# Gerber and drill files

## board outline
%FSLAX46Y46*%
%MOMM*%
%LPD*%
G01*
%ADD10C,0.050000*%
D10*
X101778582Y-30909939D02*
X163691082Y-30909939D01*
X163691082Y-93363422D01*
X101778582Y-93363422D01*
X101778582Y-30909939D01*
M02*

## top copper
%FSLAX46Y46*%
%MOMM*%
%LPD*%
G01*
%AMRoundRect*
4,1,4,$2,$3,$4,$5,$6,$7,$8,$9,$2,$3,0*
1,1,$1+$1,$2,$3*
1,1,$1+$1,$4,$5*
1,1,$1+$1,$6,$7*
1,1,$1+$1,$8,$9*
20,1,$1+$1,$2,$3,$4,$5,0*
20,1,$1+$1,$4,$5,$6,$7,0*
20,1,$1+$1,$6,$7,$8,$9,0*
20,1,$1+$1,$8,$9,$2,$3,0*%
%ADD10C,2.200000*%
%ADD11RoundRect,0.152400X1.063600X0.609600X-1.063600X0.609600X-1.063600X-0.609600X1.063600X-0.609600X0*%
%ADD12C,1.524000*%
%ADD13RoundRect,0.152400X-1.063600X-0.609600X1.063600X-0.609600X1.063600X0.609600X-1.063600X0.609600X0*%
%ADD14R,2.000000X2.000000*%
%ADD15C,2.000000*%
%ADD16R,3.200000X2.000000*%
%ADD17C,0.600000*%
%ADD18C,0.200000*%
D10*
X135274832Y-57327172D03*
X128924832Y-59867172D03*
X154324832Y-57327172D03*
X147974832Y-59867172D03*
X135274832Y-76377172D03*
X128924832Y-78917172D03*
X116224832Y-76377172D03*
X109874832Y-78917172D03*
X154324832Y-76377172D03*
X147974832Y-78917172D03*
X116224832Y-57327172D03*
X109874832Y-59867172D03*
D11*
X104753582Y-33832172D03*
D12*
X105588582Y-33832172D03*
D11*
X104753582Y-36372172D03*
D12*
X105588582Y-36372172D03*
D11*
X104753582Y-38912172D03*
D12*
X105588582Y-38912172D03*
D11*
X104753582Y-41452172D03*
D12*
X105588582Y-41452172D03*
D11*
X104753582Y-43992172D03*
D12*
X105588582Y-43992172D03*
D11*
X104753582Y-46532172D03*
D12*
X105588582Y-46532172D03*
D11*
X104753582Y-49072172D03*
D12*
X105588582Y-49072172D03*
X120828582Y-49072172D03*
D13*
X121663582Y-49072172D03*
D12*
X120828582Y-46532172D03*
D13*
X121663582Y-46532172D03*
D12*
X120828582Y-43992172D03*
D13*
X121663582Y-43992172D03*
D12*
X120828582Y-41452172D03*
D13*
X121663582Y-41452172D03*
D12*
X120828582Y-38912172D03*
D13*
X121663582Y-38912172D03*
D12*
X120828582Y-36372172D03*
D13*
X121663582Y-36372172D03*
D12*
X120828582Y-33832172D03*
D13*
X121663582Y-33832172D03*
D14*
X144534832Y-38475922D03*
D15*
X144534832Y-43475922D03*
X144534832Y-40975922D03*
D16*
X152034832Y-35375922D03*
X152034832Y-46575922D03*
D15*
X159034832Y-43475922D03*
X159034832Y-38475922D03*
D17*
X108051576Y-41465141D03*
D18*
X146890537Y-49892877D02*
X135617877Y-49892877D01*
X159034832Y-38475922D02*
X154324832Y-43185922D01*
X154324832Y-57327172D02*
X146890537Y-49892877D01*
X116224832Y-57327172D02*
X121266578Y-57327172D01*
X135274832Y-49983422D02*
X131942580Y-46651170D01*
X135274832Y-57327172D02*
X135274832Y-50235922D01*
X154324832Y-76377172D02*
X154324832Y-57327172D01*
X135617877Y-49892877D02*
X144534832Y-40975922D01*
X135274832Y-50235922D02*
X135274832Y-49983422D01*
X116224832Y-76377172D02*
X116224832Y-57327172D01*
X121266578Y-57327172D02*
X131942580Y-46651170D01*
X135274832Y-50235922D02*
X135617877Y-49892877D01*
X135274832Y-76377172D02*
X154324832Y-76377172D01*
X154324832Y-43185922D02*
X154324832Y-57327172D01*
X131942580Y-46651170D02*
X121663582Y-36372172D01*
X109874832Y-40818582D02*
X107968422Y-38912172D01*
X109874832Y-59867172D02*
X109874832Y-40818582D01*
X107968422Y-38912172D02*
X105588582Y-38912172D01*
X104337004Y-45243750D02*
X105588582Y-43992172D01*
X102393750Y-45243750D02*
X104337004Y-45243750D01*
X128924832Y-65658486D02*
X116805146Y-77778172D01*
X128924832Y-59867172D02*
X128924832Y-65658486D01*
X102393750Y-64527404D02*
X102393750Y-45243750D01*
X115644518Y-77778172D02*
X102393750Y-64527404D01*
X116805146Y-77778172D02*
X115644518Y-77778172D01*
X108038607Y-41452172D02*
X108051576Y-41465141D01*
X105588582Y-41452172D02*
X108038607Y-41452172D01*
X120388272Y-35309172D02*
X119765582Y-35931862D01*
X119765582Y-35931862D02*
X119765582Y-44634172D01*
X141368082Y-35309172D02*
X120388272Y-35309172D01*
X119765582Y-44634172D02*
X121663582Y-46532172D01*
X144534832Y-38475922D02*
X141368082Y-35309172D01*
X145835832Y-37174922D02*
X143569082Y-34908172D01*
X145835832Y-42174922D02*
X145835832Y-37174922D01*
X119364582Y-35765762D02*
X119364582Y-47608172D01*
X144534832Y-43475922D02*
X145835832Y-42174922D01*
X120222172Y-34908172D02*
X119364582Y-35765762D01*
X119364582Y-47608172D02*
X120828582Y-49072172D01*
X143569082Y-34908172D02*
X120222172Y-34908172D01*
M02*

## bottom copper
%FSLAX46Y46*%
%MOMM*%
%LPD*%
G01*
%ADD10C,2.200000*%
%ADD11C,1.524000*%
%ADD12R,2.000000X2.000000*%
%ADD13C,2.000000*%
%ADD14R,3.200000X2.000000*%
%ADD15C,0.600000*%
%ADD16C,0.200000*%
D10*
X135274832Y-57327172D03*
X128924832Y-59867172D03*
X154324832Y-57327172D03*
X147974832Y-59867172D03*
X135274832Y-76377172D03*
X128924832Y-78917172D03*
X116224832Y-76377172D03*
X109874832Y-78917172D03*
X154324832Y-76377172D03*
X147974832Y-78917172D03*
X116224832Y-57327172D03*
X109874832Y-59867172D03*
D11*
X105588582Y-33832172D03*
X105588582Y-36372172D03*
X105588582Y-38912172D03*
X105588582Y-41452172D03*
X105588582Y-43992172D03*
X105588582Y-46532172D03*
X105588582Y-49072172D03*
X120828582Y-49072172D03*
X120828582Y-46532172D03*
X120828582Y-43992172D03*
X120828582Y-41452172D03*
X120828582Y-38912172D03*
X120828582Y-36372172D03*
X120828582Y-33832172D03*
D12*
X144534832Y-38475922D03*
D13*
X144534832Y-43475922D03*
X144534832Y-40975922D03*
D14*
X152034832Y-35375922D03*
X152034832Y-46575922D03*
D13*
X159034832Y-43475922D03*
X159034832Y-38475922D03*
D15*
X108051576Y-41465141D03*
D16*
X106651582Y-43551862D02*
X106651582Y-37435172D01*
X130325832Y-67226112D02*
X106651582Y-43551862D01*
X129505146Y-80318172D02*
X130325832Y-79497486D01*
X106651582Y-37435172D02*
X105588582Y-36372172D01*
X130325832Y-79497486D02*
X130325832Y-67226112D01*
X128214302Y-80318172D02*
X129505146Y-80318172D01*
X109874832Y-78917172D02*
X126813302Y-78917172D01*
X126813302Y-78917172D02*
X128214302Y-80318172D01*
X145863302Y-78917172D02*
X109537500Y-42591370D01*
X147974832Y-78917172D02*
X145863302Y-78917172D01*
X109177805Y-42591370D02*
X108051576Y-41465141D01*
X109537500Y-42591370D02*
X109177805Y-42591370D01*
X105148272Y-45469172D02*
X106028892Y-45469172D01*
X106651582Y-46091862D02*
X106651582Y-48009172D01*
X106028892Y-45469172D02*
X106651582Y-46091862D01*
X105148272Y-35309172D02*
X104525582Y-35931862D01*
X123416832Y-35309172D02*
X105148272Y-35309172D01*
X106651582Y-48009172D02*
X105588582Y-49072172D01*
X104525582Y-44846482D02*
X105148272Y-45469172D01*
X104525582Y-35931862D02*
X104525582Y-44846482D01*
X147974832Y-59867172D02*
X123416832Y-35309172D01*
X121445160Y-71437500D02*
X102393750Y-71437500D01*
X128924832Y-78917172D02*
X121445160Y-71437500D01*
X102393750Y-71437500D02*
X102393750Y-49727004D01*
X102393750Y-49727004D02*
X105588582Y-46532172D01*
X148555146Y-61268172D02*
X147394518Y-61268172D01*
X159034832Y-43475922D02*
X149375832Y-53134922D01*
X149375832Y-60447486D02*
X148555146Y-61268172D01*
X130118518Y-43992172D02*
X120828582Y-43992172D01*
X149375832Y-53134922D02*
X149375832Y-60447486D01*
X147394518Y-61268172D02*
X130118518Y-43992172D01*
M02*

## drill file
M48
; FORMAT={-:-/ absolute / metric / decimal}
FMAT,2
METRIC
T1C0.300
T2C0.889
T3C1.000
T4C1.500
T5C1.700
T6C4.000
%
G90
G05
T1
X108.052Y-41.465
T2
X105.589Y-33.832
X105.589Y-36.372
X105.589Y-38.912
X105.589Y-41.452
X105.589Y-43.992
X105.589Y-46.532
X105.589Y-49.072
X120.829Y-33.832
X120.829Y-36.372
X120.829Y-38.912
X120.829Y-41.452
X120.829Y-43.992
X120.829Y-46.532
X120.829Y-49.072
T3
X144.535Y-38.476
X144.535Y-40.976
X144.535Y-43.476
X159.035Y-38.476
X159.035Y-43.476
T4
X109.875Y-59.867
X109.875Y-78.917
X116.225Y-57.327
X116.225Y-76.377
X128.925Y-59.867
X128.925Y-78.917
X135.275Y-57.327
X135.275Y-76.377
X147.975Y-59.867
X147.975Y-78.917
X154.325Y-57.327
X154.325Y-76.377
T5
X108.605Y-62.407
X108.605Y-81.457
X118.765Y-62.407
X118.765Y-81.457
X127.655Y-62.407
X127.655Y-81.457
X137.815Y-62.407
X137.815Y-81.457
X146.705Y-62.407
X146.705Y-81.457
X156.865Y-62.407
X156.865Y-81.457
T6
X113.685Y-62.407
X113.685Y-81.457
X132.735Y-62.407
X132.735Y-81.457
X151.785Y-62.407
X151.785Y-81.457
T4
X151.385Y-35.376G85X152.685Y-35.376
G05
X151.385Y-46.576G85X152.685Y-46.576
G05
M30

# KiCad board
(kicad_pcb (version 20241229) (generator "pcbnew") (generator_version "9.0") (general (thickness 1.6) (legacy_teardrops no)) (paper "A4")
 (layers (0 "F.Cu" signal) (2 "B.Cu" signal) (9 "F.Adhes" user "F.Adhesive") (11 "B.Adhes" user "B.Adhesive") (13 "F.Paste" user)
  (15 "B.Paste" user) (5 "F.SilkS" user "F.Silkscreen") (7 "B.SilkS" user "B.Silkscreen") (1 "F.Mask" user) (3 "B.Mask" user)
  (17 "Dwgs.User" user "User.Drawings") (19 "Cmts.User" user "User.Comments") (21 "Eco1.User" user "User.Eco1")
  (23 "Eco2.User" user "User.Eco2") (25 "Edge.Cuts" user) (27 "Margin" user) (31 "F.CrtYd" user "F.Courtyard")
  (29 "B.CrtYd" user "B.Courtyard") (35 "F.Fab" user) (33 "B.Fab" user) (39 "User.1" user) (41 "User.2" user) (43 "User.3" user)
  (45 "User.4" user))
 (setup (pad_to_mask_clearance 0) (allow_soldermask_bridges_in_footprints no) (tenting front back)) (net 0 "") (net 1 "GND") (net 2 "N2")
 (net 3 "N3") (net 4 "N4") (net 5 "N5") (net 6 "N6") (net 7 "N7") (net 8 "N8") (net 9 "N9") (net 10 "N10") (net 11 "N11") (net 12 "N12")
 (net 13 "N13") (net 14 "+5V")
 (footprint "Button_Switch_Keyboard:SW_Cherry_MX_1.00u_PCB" (layer "F.Cu") (at 135.274832 57.327172)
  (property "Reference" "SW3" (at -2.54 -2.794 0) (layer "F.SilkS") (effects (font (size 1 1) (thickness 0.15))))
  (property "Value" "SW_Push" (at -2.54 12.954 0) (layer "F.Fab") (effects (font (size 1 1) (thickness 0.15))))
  (pad "" np_thru_hole circle (at -7.62 5.08) (size 1.7 1.7) (drill 1.7) (layers "*.Cu" "*.Mask"))
  (pad "" np_thru_hole circle (at -2.54 5.08) (size 4 4) (drill 4) (layers "*.Cu" "*.Mask"))
  (pad "" np_thru_hole circle (at 2.54 5.08) (size 1.7 1.7) (drill 1.7) (layers "*.Cu" "*.Mask"))
  (pad "1" thru_hole circle (at 0 0) (size 2.2 2.2) (drill 1.5) (layers "*.Cu" "*.Mask") (remove_unused_layers no) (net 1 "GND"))
  (pad "2" thru_hole circle (at -6.35 2.54) (size 2.2 2.2) (drill 1.5) (layers "*.Cu" "*.Mask") (remove_unused_layers no) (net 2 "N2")))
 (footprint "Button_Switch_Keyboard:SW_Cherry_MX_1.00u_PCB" (layer "F.Cu") (at 154.324832 57.327172)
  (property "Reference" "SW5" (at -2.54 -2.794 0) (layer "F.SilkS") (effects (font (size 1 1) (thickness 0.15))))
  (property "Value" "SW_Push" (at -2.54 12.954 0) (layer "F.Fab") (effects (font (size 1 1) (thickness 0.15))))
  (pad "" np_thru_hole circle (at -7.62 5.08) (size 1.7 1.7) (drill 1.7) (layers "*.Cu" "*.Mask"))
  (pad "" np_thru_hole circle (at -2.54 5.08) (size 4 4) (drill 4) (layers "*.Cu" "*.Mask"))
  (pad "" np_thru_hole circle (at 2.54 5.08) (size 1.7 1.7) (drill 1.7) (layers "*.Cu" "*.Mask"))
  (pad "1" thru_hole circle (at 0 0) (size 2.2 2.2) (drill 1.5) (layers "*.Cu" "*.Mask") (remove_unused_layers no) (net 1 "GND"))
  (pad "2" thru_hole circle (at -6.35 2.54) (size 2.2 2.2) (drill 1.5) (layers "*.Cu" "*.Mask") (remove_unused_layers no) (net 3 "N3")))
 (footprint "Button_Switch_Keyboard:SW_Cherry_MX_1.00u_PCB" (layer "F.Cu") (at 135.274832 76.377172)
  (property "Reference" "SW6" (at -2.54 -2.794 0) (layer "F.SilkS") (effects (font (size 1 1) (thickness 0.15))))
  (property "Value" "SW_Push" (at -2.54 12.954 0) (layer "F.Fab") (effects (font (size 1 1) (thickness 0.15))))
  (pad "" np_thru_hole circle (at -7.62 5.08) (size 1.7 1.7) (drill 1.7) (layers "*.Cu" "*.Mask"))
  (pad "" np_thru_hole circle (at -2.54 5.08) (size 4 4) (drill 4) (layers "*.Cu" "*.Mask"))
  (pad "" np_thru_hole circle (at 2.54 5.08) (size 1.7 1.7) (drill 1.7) (layers "*.Cu" "*.Mask"))
  (pad "1" thru_hole circle (at 0 0) (size 2.2 2.2) (drill 1.5) (layers "*.Cu" "*.Mask") (remove_unused_layers no) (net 1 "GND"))
  (pad "2" thru_hole circle (at -6.35 2.54) (size 2.2 2.2) (drill 1.5) (layers "*.Cu" "*.Mask") (remove_unused_layers no) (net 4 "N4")))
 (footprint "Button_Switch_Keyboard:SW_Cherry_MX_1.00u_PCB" (layer "F.Cu") (at 116.224832 76.377172)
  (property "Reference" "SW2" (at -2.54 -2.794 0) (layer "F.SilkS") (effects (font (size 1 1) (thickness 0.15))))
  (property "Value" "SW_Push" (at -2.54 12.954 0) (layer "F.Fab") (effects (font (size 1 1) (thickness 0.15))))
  (pad "" np_thru_hole circle (at -7.62 5.08) (size 1.7 1.7) (drill 1.7) (layers "*.Cu" "*.Mask"))
  (pad "" np_thru_hole circle (at -2.54 5.08) (size 4 4) (drill 4) (layers "*.Cu" "*.Mask"))
  (pad "" np_thru_hole circle (at 2.54 5.08) (size 1.7 1.7) (drill 1.7) (layers "*.Cu" "*.Mask"))
  (pad "1" thru_hole circle (at 0 0) (size 2.2 2.2) (drill 1.5) (layers "*.Cu" "*.Mask") (remove_unused_layers no) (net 1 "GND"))
  (pad "2" thru_hole circle (at -6.35 2.54) (size 2.2 2.2) (drill 1.5) (layers "*.Cu" "*.Mask") (remove_unused_layers no) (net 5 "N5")))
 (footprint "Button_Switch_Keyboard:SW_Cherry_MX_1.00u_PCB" (layer "F.Cu") (at 154.324832 76.377172)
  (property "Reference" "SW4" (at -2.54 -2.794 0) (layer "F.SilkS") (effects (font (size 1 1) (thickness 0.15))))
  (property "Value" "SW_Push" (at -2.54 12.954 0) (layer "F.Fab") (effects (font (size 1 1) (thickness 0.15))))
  (pad "" np_thru_hole circle (at -7.62 5.08) (size 1.7 1.7) (drill 1.7) (layers "*.Cu" "*.Mask"))
  (pad "" np_thru_hole circle (at -2.54 5.08) (size 4 4) (drill 4) (layers "*.Cu" "*.Mask"))
  (pad "" np_thru_hole circle (at 2.54 5.08) (size 1.7 1.7) (drill 1.7) (layers "*.Cu" "*.Mask"))
  (pad "1" thru_hole circle (at 0 0) (size 2.2 2.2) (drill 1.5) (layers "*.Cu" "*.Mask") (remove_unused_layers no) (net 1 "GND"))
  (pad "2" thru_hole circle (at -6.35 2.54) (size 2.2 2.2) (drill 1.5) (layers "*.Cu" "*.Mask") (remove_unused_layers no) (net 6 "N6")))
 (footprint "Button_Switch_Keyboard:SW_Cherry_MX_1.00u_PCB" (layer "F.Cu") (at 116.224832 57.327172)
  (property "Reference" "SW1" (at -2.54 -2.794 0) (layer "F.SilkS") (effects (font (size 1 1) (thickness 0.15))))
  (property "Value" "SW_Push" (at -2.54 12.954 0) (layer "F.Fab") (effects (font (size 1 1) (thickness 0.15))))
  (pad "" np_thru_hole circle (at -7.62 5.08) (size 1.7 1.7) (drill 1.7) (layers "*.Cu" "*.Mask"))
  (pad "" np_thru_hole circle (at -2.54 5.08) (size 4 4) (drill 4) (layers "*.Cu" "*.Mask"))
  (pad "" np_thru_hole circle (at 2.54 5.08) (size 1.7 1.7) (drill 1.7) (layers "*.Cu" "*.Mask"))
  (pad "1" thru_hole circle (at 0 0) (size 2.2 2.2) (drill 1.5) (layers "*.Cu" "*.Mask") (remove_unused_layers no) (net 1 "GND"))
  (pad "2" thru_hole circle (at -6.35 2.54) (size 2.2 2.2) (drill 1.5) (layers "*.Cu" "*.Mask") (remove_unused_layers no) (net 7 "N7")))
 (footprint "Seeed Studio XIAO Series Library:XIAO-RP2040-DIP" (layer "F.Cu") (at 113.208582 41.452172)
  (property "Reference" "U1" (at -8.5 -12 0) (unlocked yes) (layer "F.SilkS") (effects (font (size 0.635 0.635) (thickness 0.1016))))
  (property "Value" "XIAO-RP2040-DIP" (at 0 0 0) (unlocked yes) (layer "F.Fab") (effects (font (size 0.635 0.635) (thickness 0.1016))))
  (pad "1" smd roundrect (at -8.455 -7.62 180) (size 2.432 1.524) (layers "F.Cu" "F.Mask") (roundrect_rratio 0.1) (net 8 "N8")
   (thermal_bridge_angle 45))
  (pad "1" thru_hole circle (at -7.62 -7.62 180) (size 1.524 1.524) (drill 0.889) (layers "*.Cu" "*.Mask") (remove_unused_layers no)
   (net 8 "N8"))
  (pad "2" smd roundrect (at -8.455 -5.08 180) (size 2.432 1.524) (layers "F.Cu" "F.Mask") (roundrect_rratio 0.1) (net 5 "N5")
   (thermal_bridge_angle 45))
  (pad "2" thru_hole circle (at -7.62 -5.08 180) (size 1.524 1.524) (drill 0.889) (layers "*.Cu" "*.Mask") (remove_unused_layers no)
   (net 5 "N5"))
  (pad "3" smd roundrect (at -8.455 -2.54 180) (size 2.432 1.524) (layers "F.Cu" "F.Mask") (roundrect_rratio 0.1) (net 7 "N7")
   (thermal_bridge_angle 45))
  (pad "3" thru_hole circle (at -7.62 -2.54 180) (size 1.524 1.524) (drill 0.889) (layers "*.Cu" "*.Mask") (remove_unused_layers no)
   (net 7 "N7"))
  (pad "4" smd roundrect (at -8.455 0 180) (size 2.432 1.524) (layers "F.Cu" "F.Mask") (roundrect_rratio 0.1) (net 6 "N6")
   (thermal_bridge_angle 45))
  (pad "4" thru_hole circle (at -7.62 0 180) (size 1.524 1.524) (drill 0.889) (layers "*.Cu" "*.Mask") (remove_unused_layers no)
   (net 6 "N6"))
  (pad "5" smd roundrect (at -8.455 2.54 180) (size 2.432 1.524) (layers "F.Cu" "F.Mask") (roundrect_rratio 0.1) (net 2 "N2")
   (thermal_bridge_angle 45))
  (pad "5" thru_hole circle (at -7.62 2.54 180) (size 1.524 1.524) (drill 0.889) (layers "*.Cu" "*.Mask") (remove_unused_layers no)
   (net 2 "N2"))
  (pad "6" smd roundrect (at -8.455 5.08 180) (size 2.432 1.524) (layers "F.Cu" "F.Mask") (roundrect_rratio 0.1) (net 4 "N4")
   (thermal_bridge_angle 45))
  (pad "6" thru_hole circle (at -7.62 5.08 180) (size 1.524 1.524) (drill 0.889) (layers "*.Cu" "*.Mask") (remove_unused_layers no)
   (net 4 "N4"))
  (pad "7" smd roundrect (at -8.455 7.62 180) (size 2.432 1.524) (layers "F.Cu" "F.Mask") (roundrect_rratio 0.1) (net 3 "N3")
   (thermal_bridge_angle 45))
  (pad "7" thru_hole circle (at -7.62 7.62 180) (size 1.524 1.524) (drill 0.889) (layers "*.Cu" "*.Mask") (remove_unused_layers no)
   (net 3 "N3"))
  (pad "8" thru_hole circle (at 7.62 7.62) (size 1.524 1.524) (drill 0.889) (layers "*.Cu" "*.Mask") (remove_unused_layers no) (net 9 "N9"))
  (pad "8" smd roundrect (at 8.455 7.62) (size 2.432 1.524) (layers "F.Cu" "F.Mask") (roundrect_rratio 0.1) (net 9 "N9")
   (thermal_bridge_angle 45))
  (pad "9" thru_hole circle (at 7.62 5.08) (size 1.524 1.524) (drill 0.889) (layers "*.Cu" "*.Mask") (remove_unused_layers no)
   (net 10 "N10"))
  (pad "9" smd roundrect (at 8.455 5.08) (size 2.432 1.524) (layers "F.Cu" "F.Mask") (roundrect_rratio 0.1) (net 10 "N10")
   (thermal_bridge_angle 45))
  (pad "10" thru_hole circle (at 7.62 2.54) (size 1.524 1.524) (drill 0.889) (layers "*.Cu" "*.Mask") (remove_unused_layers no)
   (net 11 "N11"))
  (pad "10" smd roundrect (at 8.455 2.54) (size 2.432 1.524) (layers "F.Cu" "F.Mask") (roundrect_rratio 0.1) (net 11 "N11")
   (thermal_bridge_angle 45))
  (pad "11" thru_hole circle (at 7.62 0) (size 1.524 1.524) (drill 0.889) (layers "*.Cu" "*.Mask") (remove_unused_layers no) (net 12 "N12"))
  (pad "11" smd roundrect (at 8.455 0) (size 2.432 1.524) (layers "F.Cu" "F.Mask") (roundrect_rratio 0.1) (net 12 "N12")
   (thermal_bridge_angle 45))
  (pad "12" thru_hole circle (at 7.62 -2.54) (size 1.524 1.524) (drill 0.889) (layers "*.Cu" "*.Mask") (remove_unused_layers no)
   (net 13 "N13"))
  (pad "12" smd roundrect (at 8.455 -2.54) (size 2.432 1.524) (layers "F.Cu" "F.Mask") (roundrect_rratio 0.1) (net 13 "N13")
   (thermal_bridge_angle 45))
  (pad "13" thru_hole circle (at 7.62 -5.08) (size 1.524 1.524) (drill 0.889) (layers "*.Cu" "*.Mask") (remove_unused_layers no)
   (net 1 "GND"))
  (pad "13" smd roundrect (at 8.455 -5.08) (size 2.432 1.524) (layers "F.Cu" "F.Mask") (roundrect_rratio 0.1) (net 1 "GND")
   (thermal_bridge_angle 45))
  (pad "14" thru_hole circle (at 7.62 -7.62) (size 1.524 1.524) (drill 0.889) (layers "*.Cu" "*.Mask") (remove_unused_layers no)
   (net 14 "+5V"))
  (pad "14" smd roundrect (at 8.455 -7.62) (size 2.432 1.524) (layers "F.Cu" "F.Mask") (roundrect_rratio 0.1) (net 14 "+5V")
   (thermal_bridge_angle 45)))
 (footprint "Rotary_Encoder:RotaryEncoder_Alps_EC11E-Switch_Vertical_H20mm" (layer "F.Cu") (at 144.534832 38.475922)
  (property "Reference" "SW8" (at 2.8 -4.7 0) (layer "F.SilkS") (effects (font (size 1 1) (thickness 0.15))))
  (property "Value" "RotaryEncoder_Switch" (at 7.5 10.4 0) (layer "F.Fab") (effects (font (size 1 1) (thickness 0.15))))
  (pad "A" thru_hole rect (at 0 0) (size 2 2) (drill 1) (layers "*.Cu" "*.Mask") (remove_unused_layers no) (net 10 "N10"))
  (pad "B" thru_hole circle (at 0 5) (size 2 2) (drill 1) (layers "*.Cu" "*.Mask") (remove_unused_layers no) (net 9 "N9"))
  (pad "C" thru_hole circle (at 0 2.5) (size 2 2) (drill 1) (layers "*.Cu" "*.Mask") (remove_unused_layers no) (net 1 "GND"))
  (pad "MP" thru_hole rect (at 7.5 -3.1) (size 3.2 2) (drill oval 2.8 1.5) (layers "*.Cu" "*.Mask") (remove_unused_layers no))
  (pad "MP" thru_hole rect (at 7.5 8.1) (size 3.2 2) (drill oval 2.8 1.5) (layers "*.Cu" "*.Mask") (remove_unused_layers no))
  (pad "S1" thru_hole circle (at 14.5 5) (size 2 2) (drill 1) (layers "*.Cu" "*.Mask") (remove_unused_layers no) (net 11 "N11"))
  (pad "S2" thru_hole circle (at 14.5 0) (size 2 2) (drill 1) (layers "*.Cu" "*.Mask") (remove_unused_layers no) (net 1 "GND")))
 (gr_rect (start 101.778582 30.909939) (end 163.691082 93.363422) (stroke (width 0.05) (type default)) (fill no) (layer "Edge.Cuts"))
 (segment (start 146.890537 49.892877) (end 135.617877 49.892877) (width 0.2) (layer "F.Cu") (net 1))
 (segment (start 159.034832 38.475922) (end 154.324832 43.185922) (width 0.2) (layer "F.Cu") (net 1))
 (segment (start 154.324832 57.327172) (end 146.890537 49.892877) (width 0.2) (layer "F.Cu") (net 1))
 (segment (start 116.224832 57.327172) (end 121.266578 57.327172) (width 0.2) (layer "F.Cu") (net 1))
 (segment (start 135.274832 49.983422) (end 131.94258 46.65117) (width 0.2) (layer "F.Cu") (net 1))
 (segment (start 135.274832 57.327172) (end 135.274832 50.235922) (width 0.2) (layer "F.Cu") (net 1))
 (segment (start 154.324832 76.377172) (end 154.324832 57.327172) (width 0.2) (layer "F.Cu") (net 1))
 (segment (start 135.617877 49.892877) (end 144.534832 40.975922) (width 0.2) (layer "F.Cu") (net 1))
 (segment (start 135.274832 50.235922) (end 135.274832 49.983422) (width 0.2) (layer "F.Cu") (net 1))
 (segment (start 116.224832 76.377172) (end 116.224832 57.327172) (width 0.2) (layer "F.Cu") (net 1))
 (segment (start 121.266578 57.327172) (end 131.94258 46.65117) (width 0.2) (layer "F.Cu") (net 1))
 (segment (start 135.274832 50.235922) (end 135.617877 49.892877) (width 0.2) (layer "F.Cu") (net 1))
 (segment (start 135.274832 76.377172) (end 154.324832 76.377172) (width 0.2) (layer "F.Cu") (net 1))
 (segment (start 154.324832 43.185922) (end 154.324832 57.327172) (width 0.2) (layer "F.Cu") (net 1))
 (segment (start 131.94258 46.65117) (end 121.663582 36.372172) (width 0.2) (layer "F.Cu") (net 1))
 (segment (start 109.874832 40.818582) (end 107.968422 38.912172) (width 0.2) (layer "F.Cu") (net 7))
 (segment (start 109.874832 59.867172) (end 109.874832 40.818582) (width 0.2) (layer "F.Cu") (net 7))
 (segment (start 107.968422 38.912172) (end 105.588582 38.912172) (width 0.2) (layer "F.Cu") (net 7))
 (segment (start 106.651582 43.551862) (end 106.651582 37.435172) (width 0.2) (layer "B.Cu") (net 5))
 (segment (start 130.325832 67.226112) (end 106.651582 43.551862) (width 0.2) (layer "B.Cu") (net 5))
 (segment (start 129.505146 80.318172) (end 130.325832 79.497486) (width 0.2) (layer "B.Cu") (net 5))
 (segment (start 106.651582 37.435172) (end 105.588582 36.372172) (width 0.2) (layer "B.Cu") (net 5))
 (segment (start 130.325832 79.497486) (end 130.325832 67.226112) (width 0.2) (layer "B.Cu") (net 5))
 (segment (start 128.214302 80.318172) (end 129.505146 80.318172) (width 0.2) (layer "B.Cu") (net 5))
 (segment (start 109.874832 78.917172) (end 126.813302 78.917172) (width 0.2) (layer "B.Cu") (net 5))
 (segment (start 126.813302 78.917172) (end 128.214302 80.318172) (width 0.2) (layer "B.Cu") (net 5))
 (segment (start 104.337004 45.24375) (end 105.588582 43.992172) (width 0.2) (layer "F.Cu") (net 2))
 (segment (start 102.39375 45.24375) (end 104.337004 45.24375) (width 0.2) (layer "F.Cu") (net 2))
 (segment (start 128.924832 65.658486) (end 116.805146 77.778172) (width 0.2) (layer "F.Cu") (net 2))
 (segment (start 128.924832 59.867172) (end 128.924832 65.658486) (width 0.2) (layer "F.Cu") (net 2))
 (segment (start 102.39375 64.527404) (end 102.39375 45.24375) (width 0.2) (layer "F.Cu") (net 2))
 (segment (start 115.644518 77.778172) (end 102.39375 64.527404) (width 0.2) (layer "F.Cu") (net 2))
 (segment (start 116.805146 77.778172) (end 115.644518 77.778172) (width 0.2) (layer "F.Cu") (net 2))
 (segment (start 108.038607 41.452172) (end 108.051576 41.465141) (width 0.2) (layer "F.Cu") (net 6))
 (segment (start 105.588582 41.452172) (end 108.038607 41.452172) (width 0.2) (layer "F.Cu") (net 6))
 (via (at 108.051576 41.465141) (size 0.6) (drill 0.3) (layers "F.Cu" "B.Cu") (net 6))
 (segment (start 145.863302 78.917172) (end 109.5375 42.59137) (width 0.2) (layer "B.Cu") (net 6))
 (segment (start 147.974832 78.917172) (end 145.863302 78.917172) (width 0.2) (layer "B.Cu") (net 6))
 (segment (start 109.177805 42.59137) (end 108.051576 41.465141) (width 0.2) (layer "B.Cu") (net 6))
 (segment (start 109.5375 42.59137) (end 109.177805 42.59137) (width 0.2) (layer "B.Cu") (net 6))
 (segment (start 105.148272 45.469172) (end 106.028892 45.469172) (width 0.2) (layer "B.Cu") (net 3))
 (segment (start 106.651582 46.091862) (end 106.651582 48.009172) (width 0.2) (layer "B.Cu") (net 3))
 (segment (start 106.028892 45.469172) (end 106.651582 46.091862) (width 0.2) (layer "B.Cu") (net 3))
 (segment (start 105.148272 35.309172) (end 104.525582 35.931862) (width 0.2) (layer "B.Cu") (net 3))
 (segment (start 123.416832 35.309172) (end 105.148272 35.309172) (width 0.2) (layer "B.Cu") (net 3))
 (segment (start 106.651582 48.009172) (end 105.588582 49.072172) (width 0.2) (layer "B.Cu") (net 3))
 (segment (start 104.525582 44.846482) (end 105.148272 45.469172) (width 0.2) (layer "B.Cu") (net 3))
 (segment (start 104.525582 35.931862) (end 104.525582 44.846482) (width 0.2) (layer "B.Cu") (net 3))
 (segment (start 147.974832 59.867172) (end 123.416832 35.309172) (width 0.2) (layer "B.Cu") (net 3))
 (segment (start 121.44516 71.4375) (end 102.39375 71.4375) (width 0.2) (layer "B.Cu") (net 4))
 (segment (start 128.924832 78.917172) (end 121.44516 71.4375) (width 0.2) (layer "B.Cu") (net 4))
 (segment (start 102.39375 71.4375) (end 102.39375 49.727004) (width 0.2) (layer "B.Cu") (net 4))
 (segment (start 102.39375 49.727004) (end 105.588582 46.532172) (width 0.2) (layer "B.Cu") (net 4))
 (segment (start 148.555146 61.268172) (end 147.394518 61.268172) (width 0.2) (layer "B.Cu") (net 11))
 (segment (start 159.034832 43.475922) (end 149.375832 53.134922) (width 0.2) (layer "B.Cu") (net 11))
 (segment (start 149.375832 60.447486) (end 148.555146 61.268172) (width 0.2) (layer "B.Cu") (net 11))
 (segment (start 130.118518 43.992172) (end 120.828582 43.992172) (width 0.2) (layer "B.Cu") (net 11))
 (segment (start 149.375832 53.134922) (end 149.375832 60.447486) (width 0.2) (layer "B.Cu") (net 11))
 (segment (start 147.394518 61.268172) (end 130.118518 43.992172) (width 0.2) (layer "B.Cu") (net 11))
 (segment (start 120.388272 35.309172) (end 119.765582 35.931862) (width 0.2) (layer "F.Cu") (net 10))
 (segment (start 119.765582 35.931862) (end 119.765582 44.634172) (width 0.2) (layer "F.Cu") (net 10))
 (segment (start 141.368082 35.309172) (end 120.388272 35.309172) (width 0.2) (layer "F.Cu") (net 10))
 (segment (start 119.765582 44.634172) (end 121.663582 46.532172) (width 0.2) (layer "F.Cu") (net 10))
 (segment (start 144.534832 38.475922) (end 141.368082 35.309172) (width 0.2) (layer "F.Cu") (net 10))
 (segment (start 145.835832 37.174922) (end 143.569082 34.908172) (width 0.2) (layer "F.Cu") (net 9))
 (segment (start 145.835832 42.174922) (end 145.835832 37.174922) (width 0.2) (layer "F.Cu") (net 9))
 (segment (start 119.364582 35.765762) (end 119.364582 47.608172) (width 0.2) (layer "F.Cu") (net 9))
 (segment (start 144.534832 43.475922) (end 145.835832 42.174922) (width 0.2) (layer "F.Cu") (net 9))
 (segment (start 120.222172 34.908172) (end 119.364582 35.765762) (width 0.2) (layer "F.Cu") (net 9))
 (segment (start 119.364582 47.608172) (end 120.828582 49.072172) (width 0.2) (layer "F.Cu") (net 9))
 (segment (start 143.569082 34.908172) (end 120.222172 34.908172) (width 0.2) (layer "F.Cu") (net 9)))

